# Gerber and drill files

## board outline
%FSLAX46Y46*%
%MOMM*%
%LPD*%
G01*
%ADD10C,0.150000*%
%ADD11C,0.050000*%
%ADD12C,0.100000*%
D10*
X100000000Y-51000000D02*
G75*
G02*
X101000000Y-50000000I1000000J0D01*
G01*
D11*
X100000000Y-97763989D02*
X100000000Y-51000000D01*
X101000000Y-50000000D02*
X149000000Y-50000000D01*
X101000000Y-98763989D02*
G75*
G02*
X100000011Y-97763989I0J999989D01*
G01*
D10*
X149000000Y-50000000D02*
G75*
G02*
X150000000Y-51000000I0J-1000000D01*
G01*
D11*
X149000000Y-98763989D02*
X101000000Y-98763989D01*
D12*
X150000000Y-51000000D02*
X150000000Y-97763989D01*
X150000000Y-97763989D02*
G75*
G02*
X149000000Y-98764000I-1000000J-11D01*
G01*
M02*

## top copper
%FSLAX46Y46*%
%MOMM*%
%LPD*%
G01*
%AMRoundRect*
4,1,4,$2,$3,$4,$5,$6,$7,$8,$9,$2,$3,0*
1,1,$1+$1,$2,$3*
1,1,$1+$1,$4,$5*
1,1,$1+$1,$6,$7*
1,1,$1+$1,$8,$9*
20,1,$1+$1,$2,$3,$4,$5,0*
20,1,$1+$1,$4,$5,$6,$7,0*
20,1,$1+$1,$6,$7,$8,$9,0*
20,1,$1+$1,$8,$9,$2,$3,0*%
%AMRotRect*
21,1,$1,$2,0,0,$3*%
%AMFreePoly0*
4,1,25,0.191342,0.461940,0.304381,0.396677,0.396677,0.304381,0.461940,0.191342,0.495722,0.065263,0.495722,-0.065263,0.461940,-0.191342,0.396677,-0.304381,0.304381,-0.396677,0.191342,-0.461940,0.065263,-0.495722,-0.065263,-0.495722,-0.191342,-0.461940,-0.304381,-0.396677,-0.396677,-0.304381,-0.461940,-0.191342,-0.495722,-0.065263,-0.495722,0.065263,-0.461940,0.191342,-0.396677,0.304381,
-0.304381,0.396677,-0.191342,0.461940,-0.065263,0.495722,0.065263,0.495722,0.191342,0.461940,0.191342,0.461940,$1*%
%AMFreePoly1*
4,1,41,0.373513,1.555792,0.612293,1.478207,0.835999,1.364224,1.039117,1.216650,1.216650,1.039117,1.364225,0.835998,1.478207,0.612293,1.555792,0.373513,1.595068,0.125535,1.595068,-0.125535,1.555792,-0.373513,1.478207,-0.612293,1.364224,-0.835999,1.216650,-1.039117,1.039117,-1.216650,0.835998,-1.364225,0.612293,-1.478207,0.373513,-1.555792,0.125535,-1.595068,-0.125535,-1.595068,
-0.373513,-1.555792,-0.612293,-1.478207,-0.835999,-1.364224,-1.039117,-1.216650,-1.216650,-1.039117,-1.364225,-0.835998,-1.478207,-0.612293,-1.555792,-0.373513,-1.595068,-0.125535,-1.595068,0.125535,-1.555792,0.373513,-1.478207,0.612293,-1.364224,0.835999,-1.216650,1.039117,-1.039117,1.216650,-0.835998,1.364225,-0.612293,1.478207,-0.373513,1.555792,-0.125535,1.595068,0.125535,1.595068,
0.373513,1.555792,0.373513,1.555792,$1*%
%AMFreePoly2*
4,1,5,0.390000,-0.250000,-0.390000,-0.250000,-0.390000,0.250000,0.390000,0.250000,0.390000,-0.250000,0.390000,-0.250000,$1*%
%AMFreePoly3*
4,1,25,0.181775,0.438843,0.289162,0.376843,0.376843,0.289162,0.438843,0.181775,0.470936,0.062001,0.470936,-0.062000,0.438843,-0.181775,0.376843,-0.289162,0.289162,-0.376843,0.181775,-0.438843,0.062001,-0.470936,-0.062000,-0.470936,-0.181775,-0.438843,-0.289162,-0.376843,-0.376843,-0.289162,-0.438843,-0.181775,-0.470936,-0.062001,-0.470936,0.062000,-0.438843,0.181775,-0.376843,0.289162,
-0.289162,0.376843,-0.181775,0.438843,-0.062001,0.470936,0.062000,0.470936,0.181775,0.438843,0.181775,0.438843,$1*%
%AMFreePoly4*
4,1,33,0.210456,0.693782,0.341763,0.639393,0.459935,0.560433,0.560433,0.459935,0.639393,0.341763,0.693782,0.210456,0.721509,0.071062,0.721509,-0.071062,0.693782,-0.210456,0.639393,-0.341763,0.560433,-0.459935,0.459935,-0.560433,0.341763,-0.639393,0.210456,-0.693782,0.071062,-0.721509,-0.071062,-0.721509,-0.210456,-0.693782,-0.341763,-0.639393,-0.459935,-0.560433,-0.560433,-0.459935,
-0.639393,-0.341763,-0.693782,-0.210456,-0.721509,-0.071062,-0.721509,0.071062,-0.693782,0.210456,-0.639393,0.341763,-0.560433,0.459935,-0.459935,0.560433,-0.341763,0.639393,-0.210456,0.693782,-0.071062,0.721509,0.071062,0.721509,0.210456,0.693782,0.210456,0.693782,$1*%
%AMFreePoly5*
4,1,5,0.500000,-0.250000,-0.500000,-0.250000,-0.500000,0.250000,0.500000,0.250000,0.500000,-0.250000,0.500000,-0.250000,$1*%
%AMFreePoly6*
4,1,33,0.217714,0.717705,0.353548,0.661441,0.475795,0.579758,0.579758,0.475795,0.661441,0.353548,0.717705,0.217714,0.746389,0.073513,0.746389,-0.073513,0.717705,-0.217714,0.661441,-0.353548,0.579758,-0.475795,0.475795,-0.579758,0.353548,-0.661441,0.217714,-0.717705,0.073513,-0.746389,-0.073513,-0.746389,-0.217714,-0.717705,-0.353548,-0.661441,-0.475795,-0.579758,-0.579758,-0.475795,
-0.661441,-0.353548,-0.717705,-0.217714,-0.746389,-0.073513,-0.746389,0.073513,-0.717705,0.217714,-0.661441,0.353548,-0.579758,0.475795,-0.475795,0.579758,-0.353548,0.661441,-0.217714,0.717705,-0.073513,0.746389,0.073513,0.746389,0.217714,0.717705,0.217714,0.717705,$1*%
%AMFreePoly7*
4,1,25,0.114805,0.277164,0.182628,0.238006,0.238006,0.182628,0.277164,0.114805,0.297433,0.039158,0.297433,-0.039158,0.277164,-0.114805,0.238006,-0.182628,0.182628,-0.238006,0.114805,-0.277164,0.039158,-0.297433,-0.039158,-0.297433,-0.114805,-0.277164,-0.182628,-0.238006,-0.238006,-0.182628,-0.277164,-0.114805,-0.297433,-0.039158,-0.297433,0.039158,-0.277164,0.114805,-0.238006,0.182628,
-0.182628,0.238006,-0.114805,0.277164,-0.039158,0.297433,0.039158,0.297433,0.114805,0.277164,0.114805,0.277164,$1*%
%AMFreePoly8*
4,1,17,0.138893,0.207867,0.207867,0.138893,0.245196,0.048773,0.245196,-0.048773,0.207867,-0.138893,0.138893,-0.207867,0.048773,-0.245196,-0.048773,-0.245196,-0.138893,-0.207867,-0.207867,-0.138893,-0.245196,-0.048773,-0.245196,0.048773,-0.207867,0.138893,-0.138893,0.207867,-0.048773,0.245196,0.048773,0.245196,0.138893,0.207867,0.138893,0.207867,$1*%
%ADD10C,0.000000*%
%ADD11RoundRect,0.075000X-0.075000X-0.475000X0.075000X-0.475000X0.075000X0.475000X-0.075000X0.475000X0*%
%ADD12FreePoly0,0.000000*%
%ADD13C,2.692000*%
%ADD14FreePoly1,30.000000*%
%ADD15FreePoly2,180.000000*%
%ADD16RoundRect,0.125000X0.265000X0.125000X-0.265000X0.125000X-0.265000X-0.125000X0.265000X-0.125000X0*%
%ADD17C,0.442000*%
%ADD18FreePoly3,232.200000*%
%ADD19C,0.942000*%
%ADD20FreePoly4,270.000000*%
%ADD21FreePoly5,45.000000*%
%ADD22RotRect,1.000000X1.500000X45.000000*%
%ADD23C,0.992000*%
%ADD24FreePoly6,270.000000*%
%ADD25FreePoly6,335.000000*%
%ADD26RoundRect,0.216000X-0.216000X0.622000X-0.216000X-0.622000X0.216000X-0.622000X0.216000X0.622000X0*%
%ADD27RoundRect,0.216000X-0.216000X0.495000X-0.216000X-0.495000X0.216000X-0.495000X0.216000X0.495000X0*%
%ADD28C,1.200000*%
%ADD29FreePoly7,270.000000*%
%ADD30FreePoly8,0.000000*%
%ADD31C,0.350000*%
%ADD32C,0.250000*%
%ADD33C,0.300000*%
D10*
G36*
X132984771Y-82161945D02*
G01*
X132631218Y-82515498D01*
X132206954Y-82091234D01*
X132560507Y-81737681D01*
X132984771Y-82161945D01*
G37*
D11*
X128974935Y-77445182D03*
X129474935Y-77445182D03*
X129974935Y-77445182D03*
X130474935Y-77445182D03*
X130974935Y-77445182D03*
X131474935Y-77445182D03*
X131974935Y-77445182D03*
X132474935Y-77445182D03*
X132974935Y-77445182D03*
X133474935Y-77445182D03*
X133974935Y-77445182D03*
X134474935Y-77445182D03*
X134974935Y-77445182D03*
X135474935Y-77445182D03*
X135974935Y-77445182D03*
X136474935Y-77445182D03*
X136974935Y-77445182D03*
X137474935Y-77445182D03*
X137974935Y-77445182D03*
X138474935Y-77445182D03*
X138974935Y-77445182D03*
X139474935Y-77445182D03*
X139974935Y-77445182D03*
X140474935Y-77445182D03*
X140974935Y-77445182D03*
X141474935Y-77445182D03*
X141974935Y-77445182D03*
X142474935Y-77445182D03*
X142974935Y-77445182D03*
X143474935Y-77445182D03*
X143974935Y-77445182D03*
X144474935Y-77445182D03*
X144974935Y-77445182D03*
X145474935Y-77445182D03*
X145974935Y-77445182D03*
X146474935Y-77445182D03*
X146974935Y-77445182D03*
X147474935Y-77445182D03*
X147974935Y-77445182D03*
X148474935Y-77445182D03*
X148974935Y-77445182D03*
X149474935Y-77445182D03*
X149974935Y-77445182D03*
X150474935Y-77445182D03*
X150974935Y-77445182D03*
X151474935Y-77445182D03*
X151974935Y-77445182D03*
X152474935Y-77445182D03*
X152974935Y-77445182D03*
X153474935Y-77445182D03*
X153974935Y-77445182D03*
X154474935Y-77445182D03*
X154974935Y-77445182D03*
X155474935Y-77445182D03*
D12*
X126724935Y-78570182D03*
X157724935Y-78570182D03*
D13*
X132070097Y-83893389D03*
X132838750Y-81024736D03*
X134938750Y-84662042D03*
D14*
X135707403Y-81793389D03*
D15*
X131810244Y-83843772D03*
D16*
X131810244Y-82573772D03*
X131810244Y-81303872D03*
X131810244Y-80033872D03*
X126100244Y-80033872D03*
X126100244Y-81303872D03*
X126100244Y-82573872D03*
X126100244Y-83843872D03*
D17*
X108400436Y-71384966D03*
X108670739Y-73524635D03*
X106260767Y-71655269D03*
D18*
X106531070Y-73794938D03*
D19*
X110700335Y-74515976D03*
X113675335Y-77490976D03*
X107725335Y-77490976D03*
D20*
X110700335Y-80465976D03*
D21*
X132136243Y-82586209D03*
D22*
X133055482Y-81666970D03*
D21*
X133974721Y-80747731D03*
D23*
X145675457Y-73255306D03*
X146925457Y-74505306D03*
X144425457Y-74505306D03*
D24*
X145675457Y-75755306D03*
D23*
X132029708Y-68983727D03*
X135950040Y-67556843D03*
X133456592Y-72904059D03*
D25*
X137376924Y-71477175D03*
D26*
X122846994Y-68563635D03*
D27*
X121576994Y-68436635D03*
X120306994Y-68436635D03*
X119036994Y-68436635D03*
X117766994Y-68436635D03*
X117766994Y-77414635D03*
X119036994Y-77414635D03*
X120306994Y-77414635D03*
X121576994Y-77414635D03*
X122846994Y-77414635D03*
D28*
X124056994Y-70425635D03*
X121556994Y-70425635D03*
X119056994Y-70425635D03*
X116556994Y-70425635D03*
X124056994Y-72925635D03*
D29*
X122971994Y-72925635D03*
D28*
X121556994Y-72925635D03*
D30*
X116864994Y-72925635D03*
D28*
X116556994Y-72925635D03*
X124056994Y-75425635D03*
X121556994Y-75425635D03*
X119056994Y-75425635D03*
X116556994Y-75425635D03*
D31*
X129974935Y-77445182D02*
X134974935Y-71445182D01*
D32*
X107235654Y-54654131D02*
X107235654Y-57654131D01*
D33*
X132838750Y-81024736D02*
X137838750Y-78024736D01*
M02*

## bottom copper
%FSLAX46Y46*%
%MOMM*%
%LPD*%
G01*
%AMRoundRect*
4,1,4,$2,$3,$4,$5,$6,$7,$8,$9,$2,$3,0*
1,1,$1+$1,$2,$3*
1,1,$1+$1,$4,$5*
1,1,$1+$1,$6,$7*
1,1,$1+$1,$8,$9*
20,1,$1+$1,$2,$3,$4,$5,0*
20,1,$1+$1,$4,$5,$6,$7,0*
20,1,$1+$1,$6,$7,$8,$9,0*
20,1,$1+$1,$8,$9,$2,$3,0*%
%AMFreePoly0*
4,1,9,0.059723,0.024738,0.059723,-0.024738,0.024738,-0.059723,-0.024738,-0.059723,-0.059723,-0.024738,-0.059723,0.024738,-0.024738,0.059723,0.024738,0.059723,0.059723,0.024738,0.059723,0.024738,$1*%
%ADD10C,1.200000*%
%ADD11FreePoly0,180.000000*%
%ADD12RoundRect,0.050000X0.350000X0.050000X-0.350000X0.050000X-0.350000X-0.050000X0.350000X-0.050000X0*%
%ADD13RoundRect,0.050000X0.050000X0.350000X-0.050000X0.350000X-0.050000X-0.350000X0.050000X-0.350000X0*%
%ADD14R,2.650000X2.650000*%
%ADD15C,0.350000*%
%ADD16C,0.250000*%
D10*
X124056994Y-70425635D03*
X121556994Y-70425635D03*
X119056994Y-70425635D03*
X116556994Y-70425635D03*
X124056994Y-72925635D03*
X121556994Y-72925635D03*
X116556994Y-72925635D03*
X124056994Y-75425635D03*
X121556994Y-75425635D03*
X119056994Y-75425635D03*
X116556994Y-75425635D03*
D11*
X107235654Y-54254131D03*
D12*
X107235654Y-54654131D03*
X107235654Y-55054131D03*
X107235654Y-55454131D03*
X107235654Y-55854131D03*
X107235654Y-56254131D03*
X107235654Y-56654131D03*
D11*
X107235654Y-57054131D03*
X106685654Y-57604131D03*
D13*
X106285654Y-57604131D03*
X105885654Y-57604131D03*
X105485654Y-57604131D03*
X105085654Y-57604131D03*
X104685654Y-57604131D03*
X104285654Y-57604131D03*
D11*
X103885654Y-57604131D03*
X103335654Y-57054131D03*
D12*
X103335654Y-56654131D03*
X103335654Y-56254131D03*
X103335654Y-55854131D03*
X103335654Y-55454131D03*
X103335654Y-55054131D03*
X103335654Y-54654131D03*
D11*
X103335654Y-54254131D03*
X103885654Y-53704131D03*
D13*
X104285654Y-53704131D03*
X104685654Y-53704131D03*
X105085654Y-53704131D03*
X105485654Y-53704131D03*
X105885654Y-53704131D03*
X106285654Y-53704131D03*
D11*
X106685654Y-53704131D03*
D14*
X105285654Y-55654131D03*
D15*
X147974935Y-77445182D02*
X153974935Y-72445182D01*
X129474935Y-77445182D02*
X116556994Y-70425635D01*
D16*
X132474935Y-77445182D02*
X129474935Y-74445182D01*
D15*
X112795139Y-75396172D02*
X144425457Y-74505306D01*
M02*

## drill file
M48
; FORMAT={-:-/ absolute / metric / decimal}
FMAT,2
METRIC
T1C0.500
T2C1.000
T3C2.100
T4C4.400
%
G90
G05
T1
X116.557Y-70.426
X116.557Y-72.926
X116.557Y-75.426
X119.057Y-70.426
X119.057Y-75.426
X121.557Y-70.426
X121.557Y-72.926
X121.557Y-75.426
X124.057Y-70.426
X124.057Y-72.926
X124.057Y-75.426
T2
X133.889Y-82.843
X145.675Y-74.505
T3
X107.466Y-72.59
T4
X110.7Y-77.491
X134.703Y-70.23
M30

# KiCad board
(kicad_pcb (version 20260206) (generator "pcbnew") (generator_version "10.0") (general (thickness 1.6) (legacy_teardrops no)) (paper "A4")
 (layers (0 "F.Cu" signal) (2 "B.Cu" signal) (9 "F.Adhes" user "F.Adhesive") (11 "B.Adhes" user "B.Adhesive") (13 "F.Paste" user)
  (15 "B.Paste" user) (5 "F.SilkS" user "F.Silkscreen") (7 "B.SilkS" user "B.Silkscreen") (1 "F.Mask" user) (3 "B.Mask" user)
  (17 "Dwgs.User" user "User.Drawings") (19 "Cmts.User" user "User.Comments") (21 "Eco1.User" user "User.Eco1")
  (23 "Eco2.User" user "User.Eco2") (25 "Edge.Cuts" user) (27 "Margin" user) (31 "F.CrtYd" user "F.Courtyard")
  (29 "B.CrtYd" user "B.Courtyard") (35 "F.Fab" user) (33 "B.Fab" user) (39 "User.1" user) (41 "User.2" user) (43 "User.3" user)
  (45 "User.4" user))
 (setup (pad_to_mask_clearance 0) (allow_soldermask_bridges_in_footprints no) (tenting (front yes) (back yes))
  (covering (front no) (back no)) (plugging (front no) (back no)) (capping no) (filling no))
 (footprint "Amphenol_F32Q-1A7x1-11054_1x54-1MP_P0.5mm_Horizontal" (layer "F.Cu") (at 142.224935 80.345182)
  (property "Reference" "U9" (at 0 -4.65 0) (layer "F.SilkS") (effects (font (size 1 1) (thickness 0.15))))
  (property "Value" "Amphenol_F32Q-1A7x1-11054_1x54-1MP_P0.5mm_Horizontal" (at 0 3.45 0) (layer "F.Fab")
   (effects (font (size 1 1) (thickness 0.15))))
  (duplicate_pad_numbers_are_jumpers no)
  (pad "1" smd roundrect (at -13.25 -2.9) (size 0.3 1.1) (layers "F.Cu" "F.Mask" "F.Paste") (roundrect_rratio 0.25))
  (pad "2" smd roundrect (at -12.75 -2.9) (size 0.3 1.1) (layers "F.Cu" "F.Mask" "F.Paste") (roundrect_rratio 0.25) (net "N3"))
  (pad "3" smd roundrect (at -12.25 -2.9) (size 0.3 1.1) (layers "F.Cu" "F.Mask" "F.Paste") (roundrect_rratio 0.25) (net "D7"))
  (pad "4" smd roundrect (at -11.75 -2.9) (size 0.3 1.1) (layers "F.Cu" "F.Mask" "F.Paste") (roundrect_rratio 0.25) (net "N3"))
  (pad "5" smd roundrect (at -11.25 -2.9) (size 0.3 1.1) (layers "F.Cu" "F.Mask" "F.Paste") (roundrect_rratio 0.25) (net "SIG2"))
  (pad "6" smd roundrect (at -10.75 -2.9) (size 0.3 1.1) (layers "F.Cu" "F.Mask" "F.Paste") (roundrect_rratio 0.25) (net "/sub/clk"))
  (pad "7" smd roundrect (at -10.25 -2.9) (size 0.3 1.1) (layers "F.Cu" "F.Mask" "F.Paste") (roundrect_rratio 0.25) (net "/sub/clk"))
  (pad "8" smd roundrect (at -9.75 -2.9) (size 0.3 1.1) (layers "F.Cu" "F.Mask" "F.Paste") (roundrect_rratio 0.25) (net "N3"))
  (pad "9" smd roundrect (at -9.25 -2.9) (size 0.3 1.1) (layers "F.Cu" "F.Mask" "F.Paste") (roundrect_rratio 0.25))
  (pad "10" smd roundrect (at -8.75 -2.9) (size 0.3 1.1) (layers "F.Cu" "F.Mask" "F.Paste") (roundrect_rratio 0.25))
  (pad "11" smd roundrect (at -8.25 -2.9) (size 0.3 1.1) (layers "F.Cu" "F.Mask" "F.Paste") (roundrect_rratio 0.25) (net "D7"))
  (pad "12" smd roundrect (at -7.75 -2.9) (size 0.3 1.1) (layers "F.Cu" "F.Mask" "F.Paste") (roundrect_rratio 0.25) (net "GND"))
  (pad "13" smd roundrect (at -7.25 -2.9) (size 0.3 1.1) (layers "F.Cu" "F.Mask" "F.Paste") (roundrect_rratio 0.25) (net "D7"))
  (pad "14" smd roundrect (at -6.75 -2.9) (size 0.3 1.1) (layers "F.Cu" "F.Mask" "F.Paste") (roundrect_rratio 0.25))
  (pad "15" smd roundrect (at -6.25 -2.9) (size 0.3 1.1) (layers "F.Cu" "F.Mask" "F.Paste") (roundrect_rratio 0.25) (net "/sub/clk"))
  (pad "16" smd roundrect (at -5.75 -2.9) (size 0.3 1.1) (layers "F.Cu" "F.Mask" "F.Paste") (roundrect_rratio 0.25))
  (pad "17" smd roundrect (at -5.25 -2.9) (size 0.3 1.1) (layers "F.Cu" "F.Mask" "F.Paste") (roundrect_rratio 0.25) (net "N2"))
  (pad "18" smd roundrect (at -4.75 -2.9) (size 0.3 1.1) (layers "F.Cu" "F.Mask" "F.Paste") (roundrect_rratio 0.25) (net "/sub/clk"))
  (pad "19" smd roundrect (at -4.25 -2.9) (size 0.3 1.1) (layers "F.Cu" "F.Mask" "F.Paste") (roundrect_rratio 0.25))
  (pad "20" smd roundrect (at -3.75 -2.9) (size 0.3 1.1) (layers "F.Cu" "F.Mask" "F.Paste") (roundrect_rratio 0.25) (clearance 0.35))
  (pad "21" smd roundrect (at -3.25 -2.9) (size 0.3 1.1) (layers "F.Cu" "F.Mask" "F.Paste") (roundrect_rratio 0.25) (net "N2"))
  (pad "22" smd roundrect (at -2.75 -2.9) (size 0.3 1.1) (layers "F.Cu" "F.Mask" "F.Paste") (roundrect_rratio 0.25) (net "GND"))
  (pad "23" smd roundrect (at -2.25 -2.9) (size 0.3 1.1) (layers "F.Cu" "F.Mask" "F.Paste") (roundrect_rratio 0.25))
  (pad "24" smd roundrect (at -1.75 -2.9) (size 0.3 1.1) (layers "F.Cu" "F.Mask" "F.Paste") (roundrect_rratio 0.25) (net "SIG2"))
  (pad "25" smd roundrect (at -1.25 -2.9) (size 0.3 1.1) (layers "F.Cu" "F.Mask" "F.Paste") (roundrect_rratio 0.25) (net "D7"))
  (pad "26" smd roundrect (at -0.75 -2.9) (size 0.3 1.1) (layers "F.Cu" "F.Mask" "F.Paste") (roundrect_rratio 0.25) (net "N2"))
  (pad "27" smd roundrect (at -0.25 -2.9) (size 0.3 1.1) (layers "F.Cu" "F.Mask" "F.Paste") (roundrect_rratio 0.25) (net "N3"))
  (pad "28" smd roundrect (at 0.25 -2.9) (size 0.3 1.1) (layers "F.Cu" "F.Mask" "F.Paste") (roundrect_rratio 0.25) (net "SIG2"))
  (pad "29" smd roundrect (at 0.75 -2.9) (size 0.3 1.1) (layers "F.Cu" "F.Mask" "F.Paste") (roundrect_rratio 0.25) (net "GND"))
  (pad "30" smd roundrect (at 1.25 -2.9) (size 0.3 1.1) (layers "F.Cu" "F.Mask" "F.Paste") (roundrect_rratio 0.25) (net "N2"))
  (pad "31" smd roundrect (at 1.75 -2.9) (size 0.3 1.1) (layers "F.Cu" "F.Mask" "F.Paste") (roundrect_rratio 0.25) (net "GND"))
  (pad "32" smd roundrect (at 2.25 -2.9) (size 0.3 1.1) (layers "F.Cu" "F.Mask" "F.Paste") (roundrect_rratio 0.25) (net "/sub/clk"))
  (pad "33" smd roundrect (at 2.75 -2.9) (size 0.3 1.1) (layers "F.Cu" "F.Mask" "F.Paste") (roundrect_rratio 0.25) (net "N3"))
  (pad "34" smd roundrect (at 3.25 -2.9) (size 0.3 1.1) (layers "F.Cu" "F.Mask" "F.Paste") (roundrect_rratio 0.25) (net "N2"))
  (pad "35" smd roundrect (at 3.75 -2.9) (size 0.3 1.1) (layers "F.Cu" "F.Mask" "F.Paste") (roundrect_rratio 0.25))
  (pad "36" smd roundrect (at 4.25 -2.9) (size 0.3 1.1) (layers "F.Cu" "F.Mask" "F.Paste") (roundrect_rratio 0.25) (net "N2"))
  (pad "37" smd roundrect (at 4.75 -2.9) (size 0.3 1.1) (layers "F.Cu" "F.Mask" "F.Paste") (roundrect_rratio 0.25) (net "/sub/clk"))
  (pad "38" smd roundrect (at 5.25 -2.9) (size 0.3 1.1) (layers "F.Cu" "F.Mask" "F.Paste") (roundrect_rratio 0.25) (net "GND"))
  (pad "39" smd roundrect (at 5.75 -2.9) (size 0.3 1.1) (layers "F.Cu" "F.Mask" "F.Paste") (roundrect_rratio 0.25) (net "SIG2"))
  (pad "40" smd roundrect (at 6.25 -2.9) (size 0.3 1.1) (layers "F.Cu" "F.Mask" "F.Paste") (roundrect_rratio 0.25) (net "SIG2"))
  (pad "41" smd roundrect (at 6.75 -2.9) (size 0.3 1.1) (layers "F.Cu" "F.Mask" "F.Paste") (roundrect_rratio 0.25) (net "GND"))
  (pad "42" smd roundrect (at 7.25 -2.9) (size 0.3 1.1) (layers "F.Cu" "F.Mask" "F.Paste") (roundrect_rratio 0.25) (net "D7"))
  (pad "43" smd roundrect (at 7.75 -2.9) (size 0.3 1.1) (layers "F.Cu" "F.Mask" "F.Paste") (roundrect_rratio 0.25) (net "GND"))
  (pad "44" smd roundrect (at 8.25 -2.9) (size 0.3 1.1) (layers "F.Cu" "F.Mask" "F.Paste") (roundrect_rratio 0.25) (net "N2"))
  (pad "45" smd roundrect (at 8.75 -2.9) (size 0.3 1.1) (layers "F.Cu" "F.Mask" "F.Paste") (roundrect_rratio 0.25) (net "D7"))
  (pad "46" smd roundrect (at 9.25 -2.9) (size 0.3 1.1) (layers "F.Cu" "F.Mask" "F.Paste") (roundrect_rratio 0.25) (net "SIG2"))
  (pad "47" smd roundrect (at 9.75 -2.9) (size 0.3 1.1) (layers "F.Cu" "F.Mask" "F.Paste") (roundrect_rratio 0.25))
  (pad "48" smd roundrect (at 10.25 -2.9) (size 0.3 1.1) (layers "F.Cu" "F.Mask" "F.Paste") (roundrect_rratio 0.25) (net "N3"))
  (pad "49" smd roundrect (at 10.75 -2.9) (size 0.3 1.1) (layers "F.Cu" "F.Mask" "F.Paste") (roundrect_rratio 0.25) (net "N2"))
  (pad "50" smd roundrect (at 11.25 -2.9) (size 0.3 1.1) (layers "F.Cu" "F.Mask" "F.Paste") (roundrect_rratio 0.25) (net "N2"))
  (pad "51" smd roundrect (at 11.75 -2.9) (size 0.3 1.1) (layers "F.Cu" "F.Mask" "F.Paste") (roundrect_rratio 0.25) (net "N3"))
  (pad "52" smd roundrect (at 12.25 -2.9) (size 0.3 1.1) (layers "F.Cu" "F.Mask" "F.Paste") (roundrect_rratio 0.25))
  (pad "53" smd roundrect (at 12.75 -2.9) (size 0.3 1.1) (layers "F.Cu" "F.Mask" "F.Paste") (roundrect_rratio 0.25) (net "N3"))
  (pad "54" smd roundrect (at 13.25 -2.9) (size 0.3 1.1) (layers "F.Cu" "F.Mask" "F.Paste") (roundrect_rratio 0.25) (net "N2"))
  (pad "MP" smd custom (at -15.5 -1.775) (size 1 1) (layers "F.Cu" "F.Mask" "F.Paste") (options (clearance outline) (anchor circle))
   (primitives))
  (pad "MP" smd custom (at 15.5 -1.775) (size 1 1) (layers "F.Cu" "F.Mask" "F.Paste") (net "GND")
   (options (clearance outline) (anchor circle)) (primitives)))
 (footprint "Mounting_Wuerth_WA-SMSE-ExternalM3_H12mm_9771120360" (layer "F.Cu") (at 133.88875 82.843389 30)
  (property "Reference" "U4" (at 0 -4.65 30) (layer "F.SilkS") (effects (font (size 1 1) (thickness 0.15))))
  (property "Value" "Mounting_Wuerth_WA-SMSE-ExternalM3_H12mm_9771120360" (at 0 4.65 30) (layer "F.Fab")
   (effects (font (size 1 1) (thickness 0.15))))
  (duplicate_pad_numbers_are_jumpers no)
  (pad "" smd custom (at 0 -2.1 30) (size 1.5 1.5) (layers "F.Paste") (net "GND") (options (clearance outline) (anchor circle)) (primitives))
  (pad "" np_thru_hole circle (at 0 0 30) (size 1 1) (drill 1) (layers "*.Cu" "*.Mask"))
  (pad "" smd custom (at 0 2.1 30) (size 1.5 1.5) (layers "F.Paste") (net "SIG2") (options (clearance outline) (anchor circle)) (primitives))
  (pad "1" smd circle (at -2.1 0 30) (size 2.692 2.692) (layers "F.Cu"))
  (pad "1" smd circle (at 0 -2.1 30) (size 2.692 2.692) (layers "F.Cu"))
  (pad "1" smd circle (at 0 2.1 30) (size 2.692 2.692) (layers "F.Cu") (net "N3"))
  (pad "1" smd custom (at 2.1 0 30) (size 3.2 3.2) (layers "F.Cu" "F.Mask") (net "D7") (options (clearance outline) (anchor circle))
   (primitives)))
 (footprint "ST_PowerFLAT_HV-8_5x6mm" (layer "F.Cu") (at 128.955244 81.938872 180)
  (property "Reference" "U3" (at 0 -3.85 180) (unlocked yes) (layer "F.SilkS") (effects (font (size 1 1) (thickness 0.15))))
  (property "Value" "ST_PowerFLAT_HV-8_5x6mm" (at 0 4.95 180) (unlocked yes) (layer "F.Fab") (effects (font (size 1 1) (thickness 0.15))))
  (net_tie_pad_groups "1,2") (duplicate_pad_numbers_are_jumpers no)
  (pad "" smd roundrect (at -2.855 -1.9049 180) (size 0.78 0.5) (layers "F.Paste") (roundrect_rratio 0.25) (thermal_bridge_angle 45))
  (pad "" smd roundrect (at -1.495 -2.04 180) (size 1.285 1.22) (layers "F.Paste") (roundrect_rratio 0.2049180328) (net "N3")
   (thermal_bridge_angle 45))
  (pad "" smd roundrect (at -1.495 -0.68 180) (size 1.285 1.22) (layers "F.Paste") (roundrect_rratio 0.2049180328) (thermal_bridge_angle 45))
  (pad "" smd roundrect (at -1.495 0.68 180) (size 1.285 1.22) (layers "F.Paste") (roundrect_rratio 0.2049180328) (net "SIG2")
   (thermal_bridge_angle 45))
  (pad "" smd roundrect (at -1.492 2.04 180) (size 1.285 1.22) (layers "F.Paste") (roundrect_rratio 0.2049180328) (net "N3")
   (thermal_bridge_angle 45))
  (pad "" smd roundrect (at -0.07 -2.04 180) (size 1.285 1.22) (layers "F.Paste") (roundrect_rratio 0.2049180328) (thermal_bridge_angle 45))
  (pad "" smd roundrect (at -0.07 -0.68 180) (size 1.285 1.22) (layers "F.Paste") (roundrect_rratio 0.2049180328) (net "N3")
   (thermal_bridge_angle 45))
  (pad "" smd roundrect (at -0.07 0.68 180) (size 1.285 1.22) (layers "F.Paste") (roundrect_rratio 0.2049180328) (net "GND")
   (thermal_bridge_angle 45))
  (pad "" smd roundrect (at -0.067 2.04 180) (size 1.285 1.22) (layers "F.Paste") (roundrect_rratio 0.2049180328) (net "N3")
   (thermal_bridge_angle 45))
  (pad "1" smd custom (at -2.855 -1.9049 180) (size 0.78 0.5) (layers "F.Cu" "F.Mask") (thermal_bridge_angle 45)
   (options (clearance outline) (anchor rect)) (primitives))
  (pad "2" smd roundrect (at -2.855 -0.6349 180) (size 0.78 0.5) (layers "F.Cu" "F.Mask" "F.Paste") (roundrect_rratio 0.25) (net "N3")
   (thermal_bridge_angle 45))
  (pad "3" smd roundrect (at -2.855 0.635 180) (size 0.78 0.5) (layers "F.Cu" "F.Mask" "F.Paste") (roundrect_rratio 0.25) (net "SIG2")
   (thermal_bridge_angle 45))
  (pad "4" smd roundrect (at -2.855 1.905 180) (size 0.78 0.5) (layers "F.Cu" "F.Mask" "F.Paste") (roundrect_rratio 0.25) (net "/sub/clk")
   (thermal_bridge_angle 45))
  (pad "5" smd roundrect (at 2.855 1.905 180) (size 0.78 0.5) (layers "F.Cu" "F.Mask" "F.Paste") (roundrect_rratio 0.25) (clearance 0.35)
   (thermal_bridge_angle 45))
  (pad "6" smd roundrect (at 2.855 0.635 180) (size 0.78 0.5) (layers "F.Cu" "F.Mask" "F.Paste") (roundrect_rratio 0.25) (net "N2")
   (clearance 0.35) (thermal_bridge_angle 45))
  (pad "7" smd roundrect (at 2.855 -0.635 180) (size 0.78 0.5) (layers "F.Cu" "F.Mask" "F.Paste") (roundrect_rratio 0.25) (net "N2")
   (thermal_bridge_angle 45))
  (pad "8" smd roundrect (at 2.855 -1.905 180) (size 0.78 0.5) (layers "F.Cu" "F.Mask" "F.Paste") (roundrect_rratio 0.25) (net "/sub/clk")
   (thermal_bridge_angle 45)))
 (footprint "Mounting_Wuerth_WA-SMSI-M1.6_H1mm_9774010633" (layer "F.Cu") (at 107.465753 72.589952 -127.8)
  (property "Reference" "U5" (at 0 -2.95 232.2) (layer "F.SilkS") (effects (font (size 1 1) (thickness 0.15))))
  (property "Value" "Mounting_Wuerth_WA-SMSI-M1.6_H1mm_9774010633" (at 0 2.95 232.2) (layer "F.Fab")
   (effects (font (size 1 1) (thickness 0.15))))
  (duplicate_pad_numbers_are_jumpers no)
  (pad "" smd custom (at -1.06066 -1.06066 232.2) (size 0.4 0.4) (layers "F.Paste") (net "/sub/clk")
   (options (clearance outline) (anchor circle)) (primitives))
  (pad "" smd custom (at -1.06066 1.06066 232.2) (size 0.4 0.4) (layers "F.Paste") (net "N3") (options (clearance outline) (anchor circle))
   (primitives))
  (pad "" np_thru_hole circle (at 0 0 232.2) (size 2.1 2.1) (drill 2.1) (layers "*.Cu" "*.Mask"))
  (pad "" smd custom (at 1.06066 -1.06066 232.2) (size 0.4 0.4) (layers "F.Paste") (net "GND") (options (clearance outline) (anchor circle))
   (primitives))
  (pad "" smd custom (at 1.06066 1.06066 232.2) (size 0.4 0.4) (layers "F.Paste") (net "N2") (options (clearance outline) (anchor circle))
   (primitives))
  (pad "1" smd circle (at -1.525 0 232.2) (size 0.442 0.442) (layers "F.Cu") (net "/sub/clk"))
  (pad "1" smd circle (at 0 -1.525 232.2) (size 0.442 0.442) (layers "F.Cu") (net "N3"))
  (pad "1" smd circle (at 0 1.525 232.2) (size 0.442 0.442) (layers "F.Cu") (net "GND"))
  (pad "1" smd custom (at 1.525 0 232.2) (size 0.95 0.95) (layers "F.Cu" "F.Mask") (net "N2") (options (clearance outline) (anchor circle))
   (primitives)))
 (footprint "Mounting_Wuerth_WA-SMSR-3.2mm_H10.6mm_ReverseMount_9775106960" (layer "F.Cu") (at 110.700335 77.490976 -90)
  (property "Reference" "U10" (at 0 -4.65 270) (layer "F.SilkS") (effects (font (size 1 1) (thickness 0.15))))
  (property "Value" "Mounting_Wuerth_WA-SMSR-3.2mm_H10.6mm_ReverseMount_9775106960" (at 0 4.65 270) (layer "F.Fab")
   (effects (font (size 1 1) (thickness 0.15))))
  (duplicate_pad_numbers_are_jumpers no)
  (pad "" smd custom (at -2.094804 -2.094804 270) (size 0.6725 0.6725) (layers "F.Paste") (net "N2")
   (options (clearance outline) (anchor circle)) (primitives))
  (pad "" smd custom (at -2.094804 2.094804 270) (size 0.6725 0.6725) (layers "F.Paste") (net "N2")
   (options (clearance outline) (anchor circle)) (primitives))
  (pad "" np_thru_hole circle (at 0 0 270) (size 4.4 4.4) (drill 4.4) (layers "*.Cu" "*.Mask"))
  (pad "" smd custom (at 2.094804 -2.094804 270) (size 0.6725 0.6725) (layers "F.Paste") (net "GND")
   (options (clearance outline) (anchor circle)) (primitives))
  (pad "" smd custom (at 2.094804 2.094804 270) (size 0.6725 0.6725) (layers "F.Paste") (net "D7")
   (options (clearance outline) (anchor circle)) (primitives))
  (pad "1" smd circle (at -2.975 0 270) (size 0.942 0.942) (layers "F.Cu"))
  (pad "1" smd circle (at 0 -2.975 270) (size 0.942 0.942) (layers "F.Cu") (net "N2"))
  (pad "1" smd circle (at 0 2.975 270) (size 0.942 0.942) (layers "F.Cu") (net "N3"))
  (pad "1" smd custom (at 2.975 0 270) (size 1.45 1.45) (layers "F.Cu" "F.Mask") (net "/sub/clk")
   (options (clearance outline) (anchor circle)) (primitives)))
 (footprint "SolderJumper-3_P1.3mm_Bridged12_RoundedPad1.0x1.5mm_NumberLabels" (layer "F.Cu") (at 133.055482 81.66697 45)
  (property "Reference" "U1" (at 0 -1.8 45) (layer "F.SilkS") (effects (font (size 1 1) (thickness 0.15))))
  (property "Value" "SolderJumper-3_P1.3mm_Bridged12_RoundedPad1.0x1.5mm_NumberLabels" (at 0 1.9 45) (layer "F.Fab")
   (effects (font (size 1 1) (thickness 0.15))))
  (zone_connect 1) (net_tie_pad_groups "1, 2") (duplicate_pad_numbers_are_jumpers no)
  (fp_poly (pts (xy -0.9 -0.3) (xy -0.4 -0.3) (xy -0.4 0.3) (xy -0.9 0.3)) (stroke (width 0) (type solid)) (fill yes) (layer "F.Cu"))
  (pad "1" smd custom (at -1.3 0 45) (size 1 0.5) (layers "F.Cu" "F.Mask") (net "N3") (zone_connect 2) (thermal_bridge_angle 45)
   (options (clearance outline) (anchor rect)) (primitives))
  (pad "2" smd rect (at 0 0 45) (size 1 1.5) (layers "F.Cu" "F.Mask") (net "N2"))
  (pad "3" smd custom (at 1.3 0 45) (size 1 0.5) (layers "F.Cu" "F.Mask") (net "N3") (zone_connect 2) (thermal_bridge_angle 45)
   (options (clearance outline) (anchor rect)) (primitives)))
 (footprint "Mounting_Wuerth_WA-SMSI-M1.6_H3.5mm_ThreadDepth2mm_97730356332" (layer "F.Cu") (at 145.675457 74.505306 -90)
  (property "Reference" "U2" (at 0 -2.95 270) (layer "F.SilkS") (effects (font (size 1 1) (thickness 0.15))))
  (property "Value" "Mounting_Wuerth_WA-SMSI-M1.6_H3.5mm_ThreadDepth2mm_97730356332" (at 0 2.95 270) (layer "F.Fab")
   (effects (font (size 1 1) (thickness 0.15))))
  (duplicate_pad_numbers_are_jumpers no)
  (pad "" smd custom (at 0 -1.25 270) (size 0.65 0.65) (layers "F.Paste") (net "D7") (options (clearance outline) (anchor circle))
   (primitives))
  (pad "" np_thru_hole circle (at 0 0 270) (size 1 1) (drill 1) (layers "*.Cu" "*.Mask"))
  (pad "" smd custom (at 0 1.25 270) (size 0.65 0.65) (layers "F.Paste") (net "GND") (options (clearance outline) (anchor circle))
   (primitives))
  (pad "1" smd circle (at -1.25 0 270) (size 0.992 0.992) (layers "F.Cu") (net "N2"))
  (pad "1" smd circle (at 0 -1.25 270) (size 0.992 0.992) (layers "F.Cu"))
  (pad "1" smd circle (at 0 1.25 270) (size 0.992 0.992) (layers "F.Cu") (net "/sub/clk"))
  (pad "1" smd custom (at 1.25 0 270) (size 1.5 1.5) (layers "F.Cu" "F.Mask") (clearance 0.35) (options (clearance outline) (anchor circle))
   (primitives)))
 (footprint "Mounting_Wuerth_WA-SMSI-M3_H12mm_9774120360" (layer "F.Cu") (at 134.703316 70.230451 -25)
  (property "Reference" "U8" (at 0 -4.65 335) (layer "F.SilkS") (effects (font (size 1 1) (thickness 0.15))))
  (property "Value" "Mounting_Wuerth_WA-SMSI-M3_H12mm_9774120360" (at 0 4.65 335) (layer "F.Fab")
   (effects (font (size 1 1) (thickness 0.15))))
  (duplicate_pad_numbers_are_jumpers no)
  (pad "" smd custom (at -2.057681 -2.057681 335) (size 0.55 0.55) (layers "F.Paste") (options (clearance outline) (anchor circle))
   (primitives))
  (pad "" smd custom (at -2.057681 2.057681 335) (size 0.55 0.55) (layers "F.Paste") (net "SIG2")
   (options (clearance outline) (anchor circle)) (primitives))
  (pad "" np_thru_hole circle (at 0 0 335) (size 4.4 4.4) (drill 4.4) (layers "*.Cu" "*.Mask"))
  (pad "" smd custom (at 2.057681 -2.057681 335) (size 0.55 0.55) (layers "F.Paste") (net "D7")
   (options (clearance outline) (anchor circle)) (primitives))
  (pad "" smd custom (at 2.057681 2.057681 335) (size 0.55 0.55) (layers "F.Paste") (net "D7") (options (clearance outline) (anchor circle))
   (primitives))
  (pad "1" smd circle (at -2.95 0 335) (size 0.992 0.992) (layers "F.Cu"))
  (pad "1" smd circle (at 0 -2.95 335) (size 0.992 0.992) (layers "F.Cu") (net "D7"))
  (pad "1" smd circle (at 0 2.95 335) (size 0.992 0.992) (layers "F.Cu") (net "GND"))
  (pad "1" smd custom (at 2.95 0 335) (size 1.5 1.5) (layers "F.Cu" "F.Mask") (options (clearance outline) (anchor circle)) (primitives)))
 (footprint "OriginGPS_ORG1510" (layer "F.Cu") (at 120.306994 72.925635 -90)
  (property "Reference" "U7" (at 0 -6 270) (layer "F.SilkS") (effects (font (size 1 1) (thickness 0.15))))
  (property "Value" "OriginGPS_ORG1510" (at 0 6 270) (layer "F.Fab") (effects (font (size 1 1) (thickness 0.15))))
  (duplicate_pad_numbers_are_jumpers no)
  (pad "1" smd roundrect (at -4.362 -2.54 270) (size 1.676 0.864) (layers "F.Cu" "F.Mask" "F.Paste") (roundrect_rratio 0.25))
  (pad "2" smd roundrect (at -4.489 -1.27 270) (size 1.422 0.864) (layers "F.Cu" "F.Mask" "F.Paste") (roundrect_rratio 0.25) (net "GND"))
  (pad "3" smd roundrect (at -4.489 0 270) (size 1.422 0.864) (layers "F.Cu" "F.Mask" "F.Paste") (roundrect_rratio 0.25) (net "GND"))
  (pad "4" smd roundrect (at -4.489 1.27 270) (size 1.422 0.864) (layers "F.Cu" "F.Mask" "F.Paste") (roundrect_rratio 0.25) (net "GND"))
  (pad "5" smd roundrect (at -4.489 2.54 270) (size 1.422 0.864) (layers "F.Cu" "F.Mask" "F.Paste") (roundrect_rratio 0.25) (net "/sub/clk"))
  (pad "6" smd roundrect (at 4.489 2.54 270) (size 1.422 0.864) (layers "F.Cu" "F.Mask" "F.Paste") (roundrect_rratio 0.25) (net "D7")
   (clearance 0.1))
  (pad "7" smd roundrect (at 4.489 1.27 270) (size 1.422 0.864) (layers "F.Cu" "F.Mask" "F.Paste") (roundrect_rratio 0.25) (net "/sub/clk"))
  (pad "8" smd roundrect (at 4.489 0 270) (size 1.422 0.864) (layers "F.Cu" "F.Mask" "F.Paste") (roundrect_rratio 0.25) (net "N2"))
  (pad "9" smd roundrect (at 4.489 -1.27 270) (size 1.422 0.864) (layers "F.Cu" "F.Mask" "F.Paste") (roundrect_rratio 0.25) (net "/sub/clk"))
  (pad "10" smd roundrect (at 4.489 -2.54 270) (size 1.422 0.864) (layers "F.Cu" "F.Mask" "F.Paste") (roundrect_rratio 0.25) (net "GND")
   (clearance 0.35))
  (pad "11" thru_hole circle (at -2.5 -3.75 270) (size 1.2 1.2) (drill 0.5) (layers "*.Cu" "B.Mask") (remove_unused_layers no) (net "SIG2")
   (clearance 0.35))
  (pad "11" thru_hole circle (at -2.5 -1.25) (size 1.2 1.2) (drill 0.5) (layers "*.Cu" "B.Mask") (remove_unused_layers no))
  (pad "11" thru_hole circle (at -2.5 1.25) (size 1.2 1.2) (drill 0.5) (layers "*.Cu" "B.Mask") (remove_unused_layers no))
  (pad "11" thru_hole circle (at -2.5 3.75) (size 1.2 1.2) (drill 0.5) (layers "*.Cu" "B.Mask") (remove_unused_layers no) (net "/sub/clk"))
  (pad "11" thru_hole circle (at 0 -3.75 270) (size 1.2 1.2) (drill 0.5) (layers "*.Cu" "B.Mask") (remove_unused_layers no) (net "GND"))
  (pad "11" smd custom (at 0 -2.665 270) (size 0.6 0.6) (layers "F.Cu") (zone_connect 0) (options (clearance outline) (anchor circle))
   (primitives))
  (pad "11" thru_hole circle (at 0 -1.25 270) (size 1.2 1.2) (drill 0.5) (layers "*.Cu" "B.Mask") (remove_unused_layers no) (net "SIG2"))
  (pad "11" smd custom (at 0 3.442) (size 0.5 0.5) (layers "F.Cu") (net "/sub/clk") (zone_connect 0)
   (options (clearance outline) (anchor circle)) (primitives))
  (pad "11" thru_hole circle (at 0 3.75 270) (size 1.2 1.2) (drill 0.5) (layers "*.Cu" "B.Mask") (remove_unused_layers no))
  (pad "11" thru_hole circle (at 2.5 -3.75 270) (size 1.2 1.2) (drill 0.5) (layers "*.Cu" "B.Mask") (remove_unused_layers no))
  (pad "11" thru_hole circle (at 2.5 -1.25 270) (size 1.2 1.2) (drill 0.5) (layers "*.Cu" "B.Mask") (remove_unused_layers no)
   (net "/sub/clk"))
  (pad "11" thru_hole circle (at 2.5 1.25 270) (size 1.2 1.2) (drill 0.5) (layers "*.Cu" "B.Mask") (remove_unused_layers no) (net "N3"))
  (pad "11" thru_hole circle (at 2.5 3.75) (size 1.2 1.2) (drill 0.5) (layers "*.Cu" "B.Mask") (remove_unused_layers no))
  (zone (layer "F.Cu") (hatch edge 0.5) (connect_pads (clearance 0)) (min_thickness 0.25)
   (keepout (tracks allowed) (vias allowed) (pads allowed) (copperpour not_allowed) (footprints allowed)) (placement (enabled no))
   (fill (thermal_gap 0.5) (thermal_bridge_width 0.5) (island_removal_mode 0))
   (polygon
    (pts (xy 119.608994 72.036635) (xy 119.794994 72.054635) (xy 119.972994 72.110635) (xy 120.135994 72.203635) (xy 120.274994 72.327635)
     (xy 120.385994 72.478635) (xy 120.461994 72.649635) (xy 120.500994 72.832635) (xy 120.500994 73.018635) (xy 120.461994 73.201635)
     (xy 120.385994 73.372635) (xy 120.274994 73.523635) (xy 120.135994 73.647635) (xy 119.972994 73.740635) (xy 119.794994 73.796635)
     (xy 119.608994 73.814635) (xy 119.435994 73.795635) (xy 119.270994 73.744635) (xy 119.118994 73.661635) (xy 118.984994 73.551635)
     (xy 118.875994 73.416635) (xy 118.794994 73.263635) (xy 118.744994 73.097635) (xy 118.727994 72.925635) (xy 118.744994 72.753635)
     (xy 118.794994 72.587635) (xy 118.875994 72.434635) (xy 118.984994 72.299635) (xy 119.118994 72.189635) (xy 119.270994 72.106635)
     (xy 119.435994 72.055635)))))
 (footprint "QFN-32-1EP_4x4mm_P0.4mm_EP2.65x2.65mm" (layer "B.Cu") (at 105.285654 55.654131 180)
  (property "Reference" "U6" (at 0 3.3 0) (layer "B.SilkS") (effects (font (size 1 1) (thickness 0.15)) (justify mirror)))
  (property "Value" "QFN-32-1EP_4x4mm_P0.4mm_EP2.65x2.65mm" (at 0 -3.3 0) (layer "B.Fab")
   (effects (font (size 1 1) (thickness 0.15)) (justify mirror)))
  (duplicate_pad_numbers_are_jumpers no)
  (pad "" smd roundrect (at -0.66 -0.66 180) (size 1.07 1.07) (layers "B.Paste") (roundrect_rratio 0.233645) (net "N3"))
  (pad "" smd roundrect (at -0.66 0.66 180) (size 1.07 1.07) (layers "B.Paste") (roundrect_rratio 0.233645) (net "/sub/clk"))
  (pad "" smd roundrect (at 0.66 -0.66 180) (size 1.07 1.07) (layers "B.Paste") (roundrect_rratio 0.233645) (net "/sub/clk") (clearance 0.1))
  (pad "" smd roundrect (at 0.66 0.66 180) (size 1.07 1.07) (layers "B.Paste") (roundrect_rratio 0.233645))
  (pad "1" smd custom (at -1.95 1.4 180) (size 0.129289 0.129289) (layers "B.Cu" "B.Mask" "B.Paste") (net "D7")
   (options (clearance outline) (anchor circle)) (primitives))
  (pad "2" smd roundrect (at -1.95 1 180) (size 0.8 0.2) (layers "B.Cu" "B.Mask" "B.Paste") (roundrect_rratio 0.25) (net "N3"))
  (pad "3" smd roundrect (at -1.95 0.6 180) (size 0.8 0.2) (layers "B.Cu" "B.Mask" "B.Paste") (roundrect_rratio 0.25))
  (pad "4" smd roundrect (at -1.95 0.2 180) (size 0.8 0.2) (layers "B.Cu" "B.Mask" "B.Paste") (roundrect_rratio 0.25))
  (pad "5" smd roundrect (at -1.95 -0.2 180) (size 0.8 0.2) (layers "B.Cu" "B.Mask" "B.Paste") (roundrect_rratio 0.25) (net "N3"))
  (pad "6" smd roundrect (at -1.95 -0.6 180) (size 0.8 0.2) (layers "B.Cu" "B.Mask" "B.Paste") (roundrect_rratio 0.25) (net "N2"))
  (pad "7" smd roundrect (at -1.95 -1 180) (size 0.8 0.2) (layers "B.Cu" "B.Mask" "B.Paste") (roundrect_rratio 0.25) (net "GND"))
  (pad "8" smd custom (at -1.95 -1.4 180) (size 0.129289 0.129289) (layers "B.Cu" "B.Mask" "B.Paste") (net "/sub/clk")
   (options (clearance outline) (anchor circle)) (primitives))
  (pad "9" smd custom (at -1.4 -1.95 180) (size 0.129289 0.129289) (layers "B.Cu" "B.Mask" "B.Paste") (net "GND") (clearance 0.35)
   (options (clearance outline) (anchor circle)) (primitives))
  (pad "10" smd roundrect (at -1 -1.95 180) (size 0.2 0.8) (layers "B.Cu" "B.Mask" "B.Paste") (roundrect_rratio 0.25) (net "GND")
   (clearance 0.35))
  (pad "11" smd roundrect (at -0.6 -1.95 180) (size 0.2 0.8) (layers "B.Cu" "B.Mask" "B.Paste") (roundrect_rratio 0.25) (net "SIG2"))
  (pad "12" smd roundrect (at -0.2 -1.95 180) (size 0.2 0.8) (layers "B.Cu" "B.Mask" "B.Paste") (roundrect_rratio 0.25) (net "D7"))
  (pad "13" smd roundrect (at 0.2 -1.95 180) (size 0.2 0.8) (layers "B.Cu" "B.Mask" "B.Paste") (roundrect_rratio 0.25) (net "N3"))
  (pad "14" smd roundrect (at 0.6 -1.95 180) (size 0.2 0.8) (layers "B.Cu" "B.Mask" "B.Paste") (roundrect_rratio 0.25))
  (pad "15" smd roundrect (at 1 -1.95 180) (size 0.2 0.8) (layers "B.Cu" "B.Mask" "B.Paste") (roundrect_rratio 0.25) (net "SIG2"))
  (pad "16" smd custom (at 1.4 -1.95 180) (size 0.129289 0.129289) (layers "B.Cu" "B.Mask" "B.Paste") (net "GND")
   (options (clearance outline) (anchor circle)) (primitives))
  (pad "17" smd custom (at 1.95 -1.4 180) (size 0.129289 0.129289) (layers "B.Cu" "B.Mask" "B.Paste") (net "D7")
   (options (clearance outline) (anchor circle)) (primitives))
  (pad "18" smd roundrect (at 1.95 -1 180) (size 0.8 0.2) (layers "B.Cu" "B.Mask" "B.Paste") (roundrect_rratio 0.25) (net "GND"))
  (pad "19" smd roundrect (at 1.95 -0.6 180) (size 0.8 0.2) (layers "B.Cu" "B.Mask" "B.Paste") (roundrect_rratio 0.25) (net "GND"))
  (pad "20" smd roundrect (at 1.95 -0.2 180) (size 0.8 0.2) (layers "B.Cu" "B.Mask" "B.Paste") (roundrect_rratio 0.25) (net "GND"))
  (pad "21" smd roundrect (at 1.95 0.2 180) (size 0.8 0.2) (layers "B.Cu" "B.Mask" "B.Paste") (roundrect_rratio 0.25))
  (pad "22" smd roundrect (at 1.95 0.6 180) (size 0.8 0.2) (layers "B.Cu" "B.Mask" "B.Paste") (roundrect_rratio 0.25))
  (pad "23" smd roundrect (at 1.95 1 180) (size 0.8 0.2) (layers "B.Cu" "B.Mask" "B.Paste") (roundrect_rratio 0.25) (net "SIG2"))
  (pad "24" smd custom (at 1.95 1.4 180) (size 0.129289 0.129289) (layers "B.Cu" "B.Mask" "B.Paste")
   (options (clearance outline) (anchor circle)) (primitives))
  (pad "25" smd custom (at 1.4 1.95 180) (size 0.129289 0.129289) (layers "B.Cu" "B.Mask" "B.Paste") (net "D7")
   (options (clearance outline) (anchor circle)) (primitives))
  (pad "26" smd roundrect (at 1 1.95 180) (size 0.2 0.8) (layers "B.Cu" "B.Mask" "B.Paste") (roundrect_rratio 0.25) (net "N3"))
  (pad "27" smd roundrect (at 0.6 1.95 180) (size 0.2 0.8) (layers "B.Cu" "B.Mask" "B.Paste") (roundrect_rratio 0.25) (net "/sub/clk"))
  (pad "28" smd roundrect (at 0.2 1.95 180) (size 0.2 0.8) (layers "B.Cu" "B.Mask" "B.Paste") (roundrect_rratio 0.25))
  (pad "29" smd roundrect (at -0.2 1.95 180) (size 0.2 0.8) (layers "B.Cu" "B.Mask" "B.Paste") (roundrect_rratio 0.25) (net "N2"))
  (pad "30" smd roundrect (at -0.6 1.95 180) (size 0.2 0.8) (layers "B.Cu" "B.Mask" "B.Paste") (roundrect_rratio 0.25))
  (pad "31" smd roundrect (at -1 1.95 180) (size 0.2 0.8) (layers "B.Cu" "B.Mask" "B.Paste") (roundrect_rratio 0.25) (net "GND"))
  (pad "32" smd custom (at -1.4 1.95 180) (size 0.129289 0.129289) (layers "B.Cu" "B.Mask" "B.Paste")
   (options (clearance outline) (anchor circle)) (primitives))
  (pad "33" smd rect (at 0 0 180) (size 2.65 2.65) (layers "B.Cu" "B.Mask") (zone_connect 2))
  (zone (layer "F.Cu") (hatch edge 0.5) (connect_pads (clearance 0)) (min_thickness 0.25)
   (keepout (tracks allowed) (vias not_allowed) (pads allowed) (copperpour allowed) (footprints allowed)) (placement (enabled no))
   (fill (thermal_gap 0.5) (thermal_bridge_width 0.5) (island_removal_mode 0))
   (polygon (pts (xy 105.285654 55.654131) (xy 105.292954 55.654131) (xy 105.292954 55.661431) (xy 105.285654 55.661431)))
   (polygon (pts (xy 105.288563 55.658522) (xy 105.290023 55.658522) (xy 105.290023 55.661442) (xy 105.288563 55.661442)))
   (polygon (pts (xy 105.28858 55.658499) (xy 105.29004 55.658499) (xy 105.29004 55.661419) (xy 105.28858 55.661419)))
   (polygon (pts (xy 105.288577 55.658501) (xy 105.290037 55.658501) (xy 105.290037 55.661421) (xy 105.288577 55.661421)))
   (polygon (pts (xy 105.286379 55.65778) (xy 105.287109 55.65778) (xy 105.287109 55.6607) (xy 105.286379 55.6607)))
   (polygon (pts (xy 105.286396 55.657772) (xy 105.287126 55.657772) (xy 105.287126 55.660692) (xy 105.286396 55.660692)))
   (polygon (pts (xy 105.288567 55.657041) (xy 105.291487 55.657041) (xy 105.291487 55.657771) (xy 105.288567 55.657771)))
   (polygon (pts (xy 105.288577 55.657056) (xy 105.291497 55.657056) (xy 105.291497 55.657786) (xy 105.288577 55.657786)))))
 (gr_arc (start 100 51) (mid 100.292893 50.292893) (end 101 50) (stroke (width 0.15) (type default)) (layer "Edge.Cuts"))
 (gr_line (start 100 97.763989) (end 100 51) (stroke (width 0.05) (type default)) (layer "Edge.Cuts"))
 (gr_line (start 101 50) (end 149 50) (stroke (width 0.05) (type default)) (layer "Edge.Cuts"))
 (gr_arc (start 101 98.763989) (mid 100.292893 98.471095) (end 100 97.763989) (stroke (width 0.05) (type default)) (layer "Edge.Cuts"))
 (gr_arc (start 149 50) (mid 149.707106 50.292893) (end 150 51) (stroke (width 0.15) (type default)) (layer "Edge.Cuts"))
 (gr_line (start 149 98.763989) (end 101 98.763989) (stroke (width 0.05) (type default)) (layer "Edge.Cuts"))
 (gr_line (start 150 51) (end 150 97.763989) (stroke (width 0.1) (type default)) (layer "Edge.Cuts"))
 (gr_arc (start 150 97.763989) (mid 149.707106 98.471095) (end 149 98.763989) (stroke (width 0.1) (type default)) (layer "Edge.Cuts"))
 (segment (start 147.974935 77.445182) (end 153.974935 72.445182) (width 0.35) (layer "B.Cu") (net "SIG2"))
 (segment (start 129.974935 77.445182) (end 134.974935 71.445182) (width 0.35) (layer "F.Cu") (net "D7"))
 (segment (start 107.235654 54.654131) (end 107.235654 57.654131) (width 0.25) (layer "F.Cu") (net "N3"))
 (segment (start 129.474935 77.445182) (end 116.556994 70.425635) (width 0.35) (layer "B.Cu") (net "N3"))
 (segment (start 132.474935 77.445182) (end 129.474935 74.445182) (width 0.25) (layer "B.Cu") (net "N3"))
 (segment (start 132.83875 81.024736) (end 137.83875 78.024736) (width 0.3) (layer "F.Cu") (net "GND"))
 (segment (start 112.795139 75.396172) (end 144.425457 74.505306) (width 0.35) (layer "B.Cu") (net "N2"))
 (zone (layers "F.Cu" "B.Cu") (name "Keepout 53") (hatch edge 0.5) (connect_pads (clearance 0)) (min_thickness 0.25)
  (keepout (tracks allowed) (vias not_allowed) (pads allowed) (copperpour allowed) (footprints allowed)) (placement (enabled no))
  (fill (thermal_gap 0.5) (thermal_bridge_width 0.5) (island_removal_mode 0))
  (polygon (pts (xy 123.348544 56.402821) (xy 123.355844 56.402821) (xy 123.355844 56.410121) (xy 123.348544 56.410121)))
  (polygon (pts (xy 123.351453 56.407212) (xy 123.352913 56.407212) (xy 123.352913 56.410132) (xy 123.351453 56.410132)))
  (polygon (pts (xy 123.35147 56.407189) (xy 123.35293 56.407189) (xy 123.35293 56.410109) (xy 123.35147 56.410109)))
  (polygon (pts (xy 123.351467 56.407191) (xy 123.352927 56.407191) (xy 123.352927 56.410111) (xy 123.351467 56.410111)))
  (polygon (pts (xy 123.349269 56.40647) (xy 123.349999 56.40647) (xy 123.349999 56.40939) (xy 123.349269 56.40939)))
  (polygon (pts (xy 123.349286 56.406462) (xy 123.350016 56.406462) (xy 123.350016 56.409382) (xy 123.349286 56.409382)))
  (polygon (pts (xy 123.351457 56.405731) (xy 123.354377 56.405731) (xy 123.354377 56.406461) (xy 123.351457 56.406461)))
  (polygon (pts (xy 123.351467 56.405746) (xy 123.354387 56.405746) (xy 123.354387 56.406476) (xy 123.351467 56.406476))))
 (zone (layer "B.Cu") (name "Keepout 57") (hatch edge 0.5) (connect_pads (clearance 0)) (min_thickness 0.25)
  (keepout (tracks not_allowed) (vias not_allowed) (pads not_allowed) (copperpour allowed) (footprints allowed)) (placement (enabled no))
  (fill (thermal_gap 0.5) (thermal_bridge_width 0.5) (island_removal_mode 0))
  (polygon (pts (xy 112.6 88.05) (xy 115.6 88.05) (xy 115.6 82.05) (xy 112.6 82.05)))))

